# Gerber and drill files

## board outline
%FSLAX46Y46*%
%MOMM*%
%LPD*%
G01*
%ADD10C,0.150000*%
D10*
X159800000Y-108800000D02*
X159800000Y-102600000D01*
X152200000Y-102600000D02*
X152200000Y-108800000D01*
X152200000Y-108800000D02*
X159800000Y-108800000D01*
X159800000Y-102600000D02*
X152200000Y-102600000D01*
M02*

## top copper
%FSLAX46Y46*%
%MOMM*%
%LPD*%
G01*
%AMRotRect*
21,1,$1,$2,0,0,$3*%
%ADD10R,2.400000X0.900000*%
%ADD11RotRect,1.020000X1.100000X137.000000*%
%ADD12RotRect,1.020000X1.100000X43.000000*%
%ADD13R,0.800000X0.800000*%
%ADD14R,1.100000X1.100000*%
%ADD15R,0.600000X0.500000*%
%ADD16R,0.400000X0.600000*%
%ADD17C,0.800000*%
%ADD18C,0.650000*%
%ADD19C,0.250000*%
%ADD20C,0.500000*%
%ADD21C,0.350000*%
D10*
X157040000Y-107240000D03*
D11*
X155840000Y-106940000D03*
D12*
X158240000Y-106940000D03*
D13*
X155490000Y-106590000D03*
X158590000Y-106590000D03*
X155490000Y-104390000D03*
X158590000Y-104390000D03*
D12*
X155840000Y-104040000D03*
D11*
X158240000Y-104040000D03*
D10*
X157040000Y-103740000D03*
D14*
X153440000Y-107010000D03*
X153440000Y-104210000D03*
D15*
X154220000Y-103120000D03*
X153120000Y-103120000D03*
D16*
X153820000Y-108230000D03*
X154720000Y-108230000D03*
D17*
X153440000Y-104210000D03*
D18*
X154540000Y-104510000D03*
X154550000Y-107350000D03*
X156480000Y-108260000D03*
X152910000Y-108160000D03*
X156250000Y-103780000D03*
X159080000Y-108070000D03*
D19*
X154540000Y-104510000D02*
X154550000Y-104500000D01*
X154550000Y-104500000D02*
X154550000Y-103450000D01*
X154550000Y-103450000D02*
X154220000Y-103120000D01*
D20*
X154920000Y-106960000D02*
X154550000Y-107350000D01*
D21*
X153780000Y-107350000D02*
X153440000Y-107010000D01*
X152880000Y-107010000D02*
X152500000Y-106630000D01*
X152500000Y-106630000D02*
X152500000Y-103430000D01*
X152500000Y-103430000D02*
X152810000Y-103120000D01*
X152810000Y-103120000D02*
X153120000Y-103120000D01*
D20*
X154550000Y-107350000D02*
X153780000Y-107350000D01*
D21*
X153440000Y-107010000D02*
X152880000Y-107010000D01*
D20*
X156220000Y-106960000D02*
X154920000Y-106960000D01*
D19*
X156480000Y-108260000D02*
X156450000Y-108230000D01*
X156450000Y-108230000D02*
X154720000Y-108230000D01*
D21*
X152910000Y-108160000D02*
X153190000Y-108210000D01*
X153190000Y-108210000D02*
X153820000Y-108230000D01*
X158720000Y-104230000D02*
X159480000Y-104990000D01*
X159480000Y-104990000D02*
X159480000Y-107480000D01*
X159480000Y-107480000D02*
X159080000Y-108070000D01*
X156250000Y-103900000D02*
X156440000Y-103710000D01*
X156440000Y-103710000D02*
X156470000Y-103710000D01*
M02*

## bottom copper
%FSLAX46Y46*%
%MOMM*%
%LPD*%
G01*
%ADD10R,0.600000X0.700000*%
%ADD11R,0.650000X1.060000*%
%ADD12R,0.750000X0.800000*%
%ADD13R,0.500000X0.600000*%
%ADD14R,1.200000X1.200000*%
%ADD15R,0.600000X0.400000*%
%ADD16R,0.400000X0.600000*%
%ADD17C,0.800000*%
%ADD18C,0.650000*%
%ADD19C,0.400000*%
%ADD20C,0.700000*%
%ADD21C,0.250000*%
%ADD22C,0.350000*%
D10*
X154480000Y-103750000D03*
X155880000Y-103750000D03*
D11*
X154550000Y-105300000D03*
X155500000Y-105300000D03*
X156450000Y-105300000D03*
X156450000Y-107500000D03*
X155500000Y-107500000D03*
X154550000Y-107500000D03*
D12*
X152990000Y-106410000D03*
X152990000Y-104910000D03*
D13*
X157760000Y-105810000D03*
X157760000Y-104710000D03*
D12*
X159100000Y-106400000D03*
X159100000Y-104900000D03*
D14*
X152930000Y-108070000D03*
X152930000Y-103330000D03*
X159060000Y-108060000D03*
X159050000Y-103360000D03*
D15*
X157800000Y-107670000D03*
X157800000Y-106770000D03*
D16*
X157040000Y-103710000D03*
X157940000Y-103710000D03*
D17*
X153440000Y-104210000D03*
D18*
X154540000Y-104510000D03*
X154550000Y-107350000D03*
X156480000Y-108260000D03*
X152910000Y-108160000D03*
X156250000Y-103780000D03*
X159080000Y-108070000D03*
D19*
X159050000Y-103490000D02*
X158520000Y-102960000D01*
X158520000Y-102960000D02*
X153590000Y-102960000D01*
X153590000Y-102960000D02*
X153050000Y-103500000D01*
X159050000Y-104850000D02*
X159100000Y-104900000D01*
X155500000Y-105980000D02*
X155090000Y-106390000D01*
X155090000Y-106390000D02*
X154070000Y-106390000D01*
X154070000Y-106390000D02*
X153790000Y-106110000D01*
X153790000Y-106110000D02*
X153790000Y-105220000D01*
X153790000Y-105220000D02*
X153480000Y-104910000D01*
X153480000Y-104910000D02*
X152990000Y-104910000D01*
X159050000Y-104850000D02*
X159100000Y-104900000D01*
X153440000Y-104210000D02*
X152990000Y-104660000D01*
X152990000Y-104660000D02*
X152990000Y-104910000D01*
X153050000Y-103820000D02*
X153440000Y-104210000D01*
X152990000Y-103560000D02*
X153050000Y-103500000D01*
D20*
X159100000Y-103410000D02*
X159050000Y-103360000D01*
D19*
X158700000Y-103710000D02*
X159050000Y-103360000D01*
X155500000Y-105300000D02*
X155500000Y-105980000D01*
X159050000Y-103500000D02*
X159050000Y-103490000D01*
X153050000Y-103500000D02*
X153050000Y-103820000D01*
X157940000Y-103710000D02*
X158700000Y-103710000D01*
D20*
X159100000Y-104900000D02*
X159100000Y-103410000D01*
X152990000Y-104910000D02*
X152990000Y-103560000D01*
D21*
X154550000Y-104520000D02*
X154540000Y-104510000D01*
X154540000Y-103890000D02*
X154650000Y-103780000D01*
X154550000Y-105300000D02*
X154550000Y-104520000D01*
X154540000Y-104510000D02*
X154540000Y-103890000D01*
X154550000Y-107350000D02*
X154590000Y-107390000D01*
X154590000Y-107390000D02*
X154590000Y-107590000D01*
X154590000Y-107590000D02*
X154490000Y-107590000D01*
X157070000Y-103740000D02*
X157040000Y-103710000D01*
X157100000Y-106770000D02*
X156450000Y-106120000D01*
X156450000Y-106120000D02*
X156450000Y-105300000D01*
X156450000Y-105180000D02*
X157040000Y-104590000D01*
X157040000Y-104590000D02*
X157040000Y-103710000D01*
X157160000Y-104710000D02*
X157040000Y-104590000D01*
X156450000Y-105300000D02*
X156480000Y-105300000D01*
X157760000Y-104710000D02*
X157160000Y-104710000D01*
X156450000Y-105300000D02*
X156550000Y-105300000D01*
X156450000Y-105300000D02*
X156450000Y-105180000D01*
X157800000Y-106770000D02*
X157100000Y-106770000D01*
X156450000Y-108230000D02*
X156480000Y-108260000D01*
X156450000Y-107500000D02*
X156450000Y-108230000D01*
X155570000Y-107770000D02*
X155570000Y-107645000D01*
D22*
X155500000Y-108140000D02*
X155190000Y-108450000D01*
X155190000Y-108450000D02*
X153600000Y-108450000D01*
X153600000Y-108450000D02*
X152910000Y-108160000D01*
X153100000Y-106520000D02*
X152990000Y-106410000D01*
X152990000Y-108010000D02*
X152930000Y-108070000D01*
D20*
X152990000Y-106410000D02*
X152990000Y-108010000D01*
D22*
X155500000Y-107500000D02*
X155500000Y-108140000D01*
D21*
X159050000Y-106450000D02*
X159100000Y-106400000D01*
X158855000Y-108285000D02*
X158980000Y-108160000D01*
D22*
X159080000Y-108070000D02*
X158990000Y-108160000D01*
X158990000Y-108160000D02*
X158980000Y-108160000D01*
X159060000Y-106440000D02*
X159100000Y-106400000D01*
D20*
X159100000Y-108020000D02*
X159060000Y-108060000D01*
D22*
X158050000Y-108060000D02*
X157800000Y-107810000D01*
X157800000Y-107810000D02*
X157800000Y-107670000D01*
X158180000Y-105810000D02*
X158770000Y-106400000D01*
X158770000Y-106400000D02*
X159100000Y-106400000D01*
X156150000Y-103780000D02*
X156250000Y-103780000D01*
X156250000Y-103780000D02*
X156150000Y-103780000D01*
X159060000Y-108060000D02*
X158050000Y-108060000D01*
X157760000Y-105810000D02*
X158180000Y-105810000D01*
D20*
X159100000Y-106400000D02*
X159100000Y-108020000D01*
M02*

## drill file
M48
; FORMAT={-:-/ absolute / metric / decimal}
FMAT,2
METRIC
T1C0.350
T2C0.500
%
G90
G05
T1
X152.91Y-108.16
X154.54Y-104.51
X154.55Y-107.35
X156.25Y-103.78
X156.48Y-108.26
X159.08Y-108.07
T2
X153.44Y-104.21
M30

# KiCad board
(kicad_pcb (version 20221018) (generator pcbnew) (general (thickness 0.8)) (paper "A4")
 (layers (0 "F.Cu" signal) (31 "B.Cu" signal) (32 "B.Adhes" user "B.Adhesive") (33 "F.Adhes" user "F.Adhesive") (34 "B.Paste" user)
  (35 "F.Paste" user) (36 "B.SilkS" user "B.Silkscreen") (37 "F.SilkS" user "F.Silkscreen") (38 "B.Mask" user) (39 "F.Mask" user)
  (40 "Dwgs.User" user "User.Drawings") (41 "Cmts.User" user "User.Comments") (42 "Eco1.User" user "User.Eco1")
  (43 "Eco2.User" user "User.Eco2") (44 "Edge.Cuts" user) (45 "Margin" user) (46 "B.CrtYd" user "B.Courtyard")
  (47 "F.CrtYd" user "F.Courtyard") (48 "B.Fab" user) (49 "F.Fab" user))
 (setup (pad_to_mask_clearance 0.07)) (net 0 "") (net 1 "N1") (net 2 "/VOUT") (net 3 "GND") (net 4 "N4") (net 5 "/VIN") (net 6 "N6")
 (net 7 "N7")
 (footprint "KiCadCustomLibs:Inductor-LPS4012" (layer "F.Cu") (at 157.04 105.49 90)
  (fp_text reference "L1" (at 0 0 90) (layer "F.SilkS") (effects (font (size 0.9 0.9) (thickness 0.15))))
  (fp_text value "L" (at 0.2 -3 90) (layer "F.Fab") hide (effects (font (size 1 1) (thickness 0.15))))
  (pad "1" smd rect (at -1.75 0 90) (size 0.9 2.4) (layers "F.Cu" "F.Paste" "F.Mask") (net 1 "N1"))
  (pad "1" smd rect (at -1.45 -1.2 137) (size 1.02 1.1) (layers "F.Cu" "F.Paste" "F.Mask") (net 1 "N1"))
  (pad "1" smd rect (at -1.45 1.2 43) (size 1.02 1.1) (layers "F.Cu" "F.Paste" "F.Mask") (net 1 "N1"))
  (pad "1" smd rect (at -1.1 -1.55 90) (size 0.8 0.8) (layers "F.Cu" "F.Paste" "F.Mask") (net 1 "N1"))
  (pad "1" smd rect (at -1.1 1.55 90) (size 0.8 0.8) (layers "F.Cu" "F.Paste" "F.Mask") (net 1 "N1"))
  (pad "2" smd rect (at 1.1 -1.55 90) (size 0.8 0.8) (layers "F.Cu" "F.Paste" "F.Mask") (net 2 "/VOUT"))
  (pad "2" smd rect (at 1.1 1.55 90) (size 0.8 0.8) (layers "F.Cu" "F.Paste" "F.Mask") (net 2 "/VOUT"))
  (pad "2" smd rect (at 1.45 -1.2 43) (size 1.02 1.1) (layers "F.Cu" "F.Paste" "F.Mask") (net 2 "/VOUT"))
  (pad "2" smd rect (at 1.45 1.2 137) (size 1.02 1.1) (layers "F.Cu" "F.Paste" "F.Mask") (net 2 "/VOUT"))
  (pad "2" smd rect (at 1.75 0 90) (size 0.9 2.4) (layers "F.Cu" "F.Paste" "F.Mask") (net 2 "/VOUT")))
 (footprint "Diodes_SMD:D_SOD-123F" (layer "F.Cu") (at 153.44 105.61 90)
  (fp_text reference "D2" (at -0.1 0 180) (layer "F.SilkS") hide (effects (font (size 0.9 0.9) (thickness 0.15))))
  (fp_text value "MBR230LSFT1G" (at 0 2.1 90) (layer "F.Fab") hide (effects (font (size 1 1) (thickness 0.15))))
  (pad "1" smd rect (at -1.4 0 90) (size 1.1 1.1) (layers "F.Cu" "F.Paste" "F.Mask") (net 1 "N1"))
  (pad "2" smd rect (at 1.4 0 90) (size 1.1 1.1) (layers "F.Cu" "F.Paste" "F.Mask") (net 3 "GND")))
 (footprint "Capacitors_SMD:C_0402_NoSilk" (layer "F.Cu") (at 153.67 103.12 180)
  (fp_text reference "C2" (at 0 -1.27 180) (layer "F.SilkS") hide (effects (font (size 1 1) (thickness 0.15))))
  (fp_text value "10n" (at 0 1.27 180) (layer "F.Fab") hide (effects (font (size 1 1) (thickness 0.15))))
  (pad "1" smd rect (at -0.55 0 180) (size 0.6 0.5) (layers "F.Cu" "F.Paste" "F.Mask") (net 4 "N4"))
  (pad "2" smd rect (at 0.55 0 180) (size 0.6 0.5) (layers "F.Cu" "F.Paste" "F.Mask") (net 1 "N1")))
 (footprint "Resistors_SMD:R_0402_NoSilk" (layer "F.Cu") (at 154.27 108.23)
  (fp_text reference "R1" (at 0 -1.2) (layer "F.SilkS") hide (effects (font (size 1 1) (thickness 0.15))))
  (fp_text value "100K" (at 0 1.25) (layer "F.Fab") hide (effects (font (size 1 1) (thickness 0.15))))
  (pad "1" smd rect (at -0.45 0) (size 0.4 0.6) (layers "F.Cu" "F.Paste" "F.Mask") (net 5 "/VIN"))
  (pad "2" smd rect (at 0.45 0) (size 0.4 0.6) (layers "F.Cu" "F.Paste" "F.Mask") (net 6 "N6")))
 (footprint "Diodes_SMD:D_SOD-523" (layer "B.Cu") (at 155.18 103.75)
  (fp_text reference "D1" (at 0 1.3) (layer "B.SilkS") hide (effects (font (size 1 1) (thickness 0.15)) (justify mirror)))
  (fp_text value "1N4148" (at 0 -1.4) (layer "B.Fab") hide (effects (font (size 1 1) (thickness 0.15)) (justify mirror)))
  (pad "1" smd rect (at -0.7 0 180) (size 0.6 0.7) (layers "B.Cu" "B.Paste" "B.Mask") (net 4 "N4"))
  (pad "2" smd rect (at 0.7 0 180) (size 0.6 0.7) (layers "B.Cu" "B.Paste" "B.Mask") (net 2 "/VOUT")))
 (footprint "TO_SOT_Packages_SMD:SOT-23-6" (layer "B.Cu") (at 155.5 106.4 -90)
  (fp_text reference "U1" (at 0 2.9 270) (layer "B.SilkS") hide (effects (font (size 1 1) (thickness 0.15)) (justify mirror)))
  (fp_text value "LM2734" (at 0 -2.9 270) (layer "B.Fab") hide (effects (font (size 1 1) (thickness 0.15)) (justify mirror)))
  (pad "1" smd rect (at -1.1 0.95 270) (size 1.06 0.65) (layers "B.Cu" "B.Paste" "B.Mask") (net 4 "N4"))
  (pad "2" smd rect (at -1.1 0 270) (size 1.06 0.65) (layers "B.Cu" "B.Paste" "B.Mask") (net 3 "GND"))
  (pad "3" smd rect (at -1.1 -0.95 270) (size 1.06 0.65) (layers "B.Cu" "B.Paste" "B.Mask") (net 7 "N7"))
  (pad "4" smd rect (at 1.1 -0.95 270) (size 1.06 0.65) (layers "B.Cu" "B.Paste" "B.Mask") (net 6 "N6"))
  (pad "5" smd rect (at 1.1 0 270) (size 1.06 0.65) (layers "B.Cu" "B.Paste" "B.Mask") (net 5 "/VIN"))
  (pad "6" smd rect (at 1.1 0.95 270) (size 1.06 0.65) (layers "B.Cu" "B.Paste" "B.Mask") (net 1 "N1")))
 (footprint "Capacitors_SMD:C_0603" (layer "B.Cu") (at 152.99 105.66 90)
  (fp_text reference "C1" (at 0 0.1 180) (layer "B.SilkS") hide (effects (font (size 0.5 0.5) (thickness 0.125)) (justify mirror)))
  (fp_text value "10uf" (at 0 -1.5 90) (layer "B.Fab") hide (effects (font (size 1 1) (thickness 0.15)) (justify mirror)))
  (pad "1" smd rect (at -0.75 0 90) (size 0.8 0.75) (layers "B.Cu" "B.Paste" "B.Mask") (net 5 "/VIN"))
  (pad "2" smd rect (at 0.75 0 90) (size 0.8 0.75) (layers "B.Cu" "B.Paste" "B.Mask") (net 3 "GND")))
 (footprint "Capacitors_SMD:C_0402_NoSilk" (layer "B.Cu") (at 157.76 105.26 90)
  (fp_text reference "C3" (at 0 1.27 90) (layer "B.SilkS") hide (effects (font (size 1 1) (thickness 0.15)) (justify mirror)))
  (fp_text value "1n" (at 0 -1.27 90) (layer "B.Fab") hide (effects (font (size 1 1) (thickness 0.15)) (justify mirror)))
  (pad "1" smd rect (at -0.55 0 90) (size 0.6 0.5) (layers "B.Cu" "B.Paste" "B.Mask") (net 2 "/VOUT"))
  (pad "2" smd rect (at 0.55 0 90) (size 0.6 0.5) (layers "B.Cu" "B.Paste" "B.Mask") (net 7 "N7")))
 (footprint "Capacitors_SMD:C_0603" (layer "B.Cu") (at 159.1 105.65 90)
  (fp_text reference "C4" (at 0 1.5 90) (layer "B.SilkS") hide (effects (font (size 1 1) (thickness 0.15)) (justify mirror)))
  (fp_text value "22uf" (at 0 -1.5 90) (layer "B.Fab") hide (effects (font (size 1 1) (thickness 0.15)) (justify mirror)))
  (pad "1" smd rect (at -0.75 0 90) (size 0.8 0.75) (layers "B.Cu" "B.Paste" "B.Mask") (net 2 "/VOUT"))
  (pad "2" smd rect (at 0.75 0 90) (size 0.8 0.75) (layers "B.Cu" "B.Paste" "B.Mask") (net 3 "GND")))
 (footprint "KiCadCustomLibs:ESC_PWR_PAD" (layer "B.Cu") (at 152.93 108.07)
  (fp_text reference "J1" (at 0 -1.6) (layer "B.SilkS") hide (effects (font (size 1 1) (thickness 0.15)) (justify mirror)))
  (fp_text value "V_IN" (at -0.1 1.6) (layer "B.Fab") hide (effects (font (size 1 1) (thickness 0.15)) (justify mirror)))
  (pad "1" smd rect (at 0 0) (size 1.2 1.2) (layers "B.Cu" "B.Paste" "B.Mask") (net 5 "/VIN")))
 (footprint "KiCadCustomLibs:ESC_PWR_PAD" (layer "B.Cu") (at 152.93 103.33)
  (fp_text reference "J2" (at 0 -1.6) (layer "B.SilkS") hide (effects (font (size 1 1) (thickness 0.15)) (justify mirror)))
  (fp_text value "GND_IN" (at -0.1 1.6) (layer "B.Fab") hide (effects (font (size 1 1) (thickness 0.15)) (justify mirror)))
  (pad "1" smd rect (at 0 0) (size 1.2 1.2) (layers "B.Cu" "B.Paste" "B.Mask") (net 3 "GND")))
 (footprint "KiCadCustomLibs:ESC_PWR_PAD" (layer "B.Cu") (at 159.06 108.06)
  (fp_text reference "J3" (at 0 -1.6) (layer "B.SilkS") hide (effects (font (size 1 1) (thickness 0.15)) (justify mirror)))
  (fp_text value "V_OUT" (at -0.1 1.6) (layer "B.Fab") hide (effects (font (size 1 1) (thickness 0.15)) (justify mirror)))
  (pad "1" smd rect (at 0 0) (size 1.2 1.2) (layers "B.Cu" "B.Paste" "B.Mask") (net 2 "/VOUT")))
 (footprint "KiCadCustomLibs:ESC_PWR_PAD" (layer "B.Cu") (at 159.05 103.36)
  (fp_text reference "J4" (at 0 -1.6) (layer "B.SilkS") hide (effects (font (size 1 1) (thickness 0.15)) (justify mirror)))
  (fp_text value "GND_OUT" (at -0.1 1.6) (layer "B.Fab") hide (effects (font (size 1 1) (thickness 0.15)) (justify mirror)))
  (pad "1" smd rect (at 0 0) (size 1.2 1.2) (layers "B.Cu" "B.Paste" "B.Mask") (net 3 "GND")))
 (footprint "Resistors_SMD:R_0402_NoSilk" (layer "B.Cu") (at 157.8 107.22 90)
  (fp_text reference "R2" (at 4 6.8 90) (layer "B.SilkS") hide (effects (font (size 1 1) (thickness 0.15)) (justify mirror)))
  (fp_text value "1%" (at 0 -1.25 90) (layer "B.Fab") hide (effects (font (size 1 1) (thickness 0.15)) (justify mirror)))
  (pad "1" smd rect (at -0.45 0 90) (size 0.4 0.6) (layers "B.Cu" "B.Paste" "B.Mask") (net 2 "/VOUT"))
  (pad "2" smd rect (at 0.45 0 90) (size 0.4 0.6) (layers "B.Cu" "B.Paste" "B.Mask") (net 7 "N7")))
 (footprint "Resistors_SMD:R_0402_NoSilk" (layer "B.Cu") (at 157.49 103.71)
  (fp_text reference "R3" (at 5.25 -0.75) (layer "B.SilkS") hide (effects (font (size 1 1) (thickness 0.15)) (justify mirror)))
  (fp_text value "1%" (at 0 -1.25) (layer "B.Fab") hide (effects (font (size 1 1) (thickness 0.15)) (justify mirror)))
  (pad "1" smd rect (at -0.45 0) (size 0.4 0.6) (layers "B.Cu" "B.Paste" "B.Mask") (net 7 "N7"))
  (pad "2" smd rect (at 0.45 0) (size 0.4 0.6) (layers "B.Cu" "B.Paste" "B.Mask") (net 3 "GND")))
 (gr_line (start 159.8 108.8) (end 159.8 102.6) (stroke (width 0.15) (type solid)) (layer "Edge.Cuts"))
 (gr_line (start 152.2 102.6) (end 152.2 108.8) (stroke (width 0.15) (type solid)) (layer "Edge.Cuts"))
 (gr_line (start 152.2 108.8) (end 159.8 108.8) (stroke (width 0.15) (type solid)) (layer "Edge.Cuts"))
 (gr_line (start 159.8 102.6) (end 152.2 102.6) (stroke (width 0.15) (type solid)) (layer "Edge.Cuts"))
 (via (at 153.44 104.21) (size 0.8) (drill 0.5) (layers "F.Cu" "B.Cu") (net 3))
 (segment (start 159.05 103.49) (end 158.52 102.96) (width 0.4) (layer "B.Cu") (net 3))
 (segment (start 158.52 102.96) (end 153.59 102.96) (width 0.4) (layer "B.Cu") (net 3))
 (segment (start 153.59 102.96) (end 153.05 103.5) (width 0.4) (layer "B.Cu") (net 3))
 (segment (start 159.05 104.85) (end 159.1 104.9) (width 0.4) (layer "B.Cu") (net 3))
 (segment (start 155.5 105.98) (end 155.09 106.39) (width 0.4) (layer "B.Cu") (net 3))
 (segment (start 155.09 106.39) (end 154.07 106.39) (width 0.4) (layer "B.Cu") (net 3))
 (segment (start 154.07 106.39) (end 153.79 106.11) (width 0.4) (layer "B.Cu") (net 3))
 (segment (start 153.79 106.11) (end 153.79 105.22) (width 0.4) (layer "B.Cu") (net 3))
 (segment (start 153.79 105.22) (end 153.48 104.91) (width 0.4) (layer "B.Cu") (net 3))
 (segment (start 153.48 104.91) (end 152.99 104.91) (width 0.4) (layer "B.Cu") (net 3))
 (segment (start 159.05 104.85) (end 159.1 104.9) (width 0.4) (layer "B.Cu") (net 3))
 (segment (start 153.44 104.21) (end 152.99 104.66) (width 0.4) (layer "B.Cu") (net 3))
 (segment (start 152.99 104.66) (end 152.99 104.91) (width 0.4) (layer "B.Cu") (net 3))
 (segment (start 153.05 103.82) (end 153.44 104.21) (width 0.4) (layer "B.Cu") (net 3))
 (segment (start 152.99 103.56) (end 153.05 103.5) (width 0.4) (layer "B.Cu") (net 3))
 (segment (start 159.1 103.41) (end 159.05 103.36) (width 0.7) (layer "B.Cu") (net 3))
 (segment (start 158.7 103.71) (end 159.05 103.36) (width 0.4) (layer "B.Cu") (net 3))
 (segment (start 155.5 105.3) (end 155.5 105.98) (width 0.4) (layer "B.Cu") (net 3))
 (segment (start 159.05 103.5) (end 159.05 103.49) (width 0.4) (layer "B.Cu") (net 3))
 (segment (start 153.05 103.5) (end 153.05 103.82) (width 0.4) (layer "B.Cu") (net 3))
 (segment (start 157.94 103.71) (end 158.7 103.71) (width 0.4) (layer "B.Cu") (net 3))
 (segment (start 159.1 104.9) (end 159.1 103.41) (width 0.7) (layer "B.Cu") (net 3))
 (segment (start 152.99 104.91) (end 152.99 103.56) (width 0.7) (layer "B.Cu") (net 3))
 (segment (start 154.54 104.51) (end 154.55 104.5) (width 0.25) (layer "F.Cu") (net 4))
 (segment (start 154.55 104.5) (end 154.55 103.45) (width 0.25) (layer "F.Cu") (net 4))
 (segment (start 154.55 103.45) (end 154.22 103.12) (width 0.25) (layer "F.Cu") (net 4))
 (via (at 154.54 104.51) (size 0.65) (drill 0.35) (layers "F.Cu" "B.Cu") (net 4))
 (segment (start 154.55 104.52) (end 154.54 104.51) (width 0.25) (layer "B.Cu") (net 4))
 (segment (start 154.54 103.89) (end 154.65 103.78) (width 0.25) (layer "B.Cu") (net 4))
 (segment (start 154.55 105.3) (end 154.55 104.52) (width 0.25) (layer "B.Cu") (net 4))
 (segment (start 154.54 104.51) (end 154.54 103.89) (width 0.25) (layer "B.Cu") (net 4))
 (segment (start 154.92 106.96) (end 154.55 107.35) (width 0.5) (layer "F.Cu") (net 1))
 (segment (start 153.78 107.35) (end 153.44 107.01) (width 0.35) (layer "F.Cu") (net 1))
 (segment (start 152.88 107.01) (end 152.5 106.63) (width 0.35) (layer "F.Cu") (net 1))
 (segment (start 152.5 106.63) (end 152.5 103.43) (width 0.35) (layer "F.Cu") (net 1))
 (segment (start 152.5 103.43) (end 152.81 103.12) (width 0.35) (layer "F.Cu") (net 1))
 (segment (start 152.81 103.12) (end 153.12 103.12) (width 0.35) (layer "F.Cu") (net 1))
 (segment (start 154.55 107.35) (end 153.78 107.35) (width 0.5) (layer "F.Cu") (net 1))
 (segment (start 153.44 107.01) (end 152.88 107.01) (width 0.35) (layer "F.Cu") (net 1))
 (segment (start 156.22 106.96) (end 154.92 106.96) (width 0.5) (layer "F.Cu") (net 1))
 (via (at 154.55 107.35) (size 0.65) (drill 0.35) (layers "F.Cu" "B.Cu") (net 1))
 (segment (start 154.55 107.35) (end 154.59 107.39) (width 0.25) (layer "B.Cu") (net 1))
 (segment (start 154.59 107.39) (end 154.59 107.59) (width 0.25) (layer "B.Cu") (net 1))
 (segment (start 154.59 107.59) (end 154.49 107.59) (width 0.25) (layer "B.Cu") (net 1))
 (segment (start 157.07 103.74) (end 157.04 103.71) (width 0.25) (layer "B.Cu") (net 7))
 (segment (start 157.1 106.77) (end 156.45 106.12) (width 0.25) (layer "B.Cu") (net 7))
 (segment (start 156.45 106.12) (end 156.45 105.3) (width 0.25) (layer "B.Cu") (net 7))
 (segment (start 156.45 105.18) (end 157.04 104.59) (width 0.25) (layer "B.Cu") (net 7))
 (segment (start 157.04 104.59) (end 157.04 103.71) (width 0.25) (layer "B.Cu") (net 7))
 (segment (start 157.16 104.71) (end 157.04 104.59) (width 0.25) (layer "B.Cu") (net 7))
 (segment (start 156.45 105.3) (end 156.48 105.3) (width 0.25) (layer "B.Cu") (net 7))
 (segment (start 157.76 104.71) (end 157.16 104.71) (width 0.25) (layer "B.Cu") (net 7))
 (segment (start 156.45 105.3) (end 156.55 105.3) (width 0.25) (layer "B.Cu") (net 7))
 (segment (start 156.45 105.3) (end 156.45 105.18) (width 0.25) (layer "B.Cu") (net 7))
 (segment (start 157.8 106.77) (end 157.1 106.77) (width 0.25) (layer "B.Cu") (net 7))
 (segment (start 156.48 108.26) (end 156.45 108.23) (width 0.25) (layer "F.Cu") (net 6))
 (segment (start 156.45 108.23) (end 154.72 108.23) (width 0.25) (layer "F.Cu") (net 6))
 (via (at 156.48 108.26) (size 0.65) (drill 0.35) (layers "F.Cu" "B.Cu") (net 6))
 (segment (start 156.45 108.23) (end 156.48 108.26) (width 0.25) (layer "B.Cu") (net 6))
 (segment (start 156.45 107.5) (end 156.45 108.23) (width 0.25) (layer "B.Cu") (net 6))
 (segment (start 152.91 108.16) (end 153.19 108.21) (width 0.35) (layer "F.Cu") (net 5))
 (segment (start 153.19 108.21) (end 153.82 108.23) (width 0.35) (layer "F.Cu") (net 5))
 (via (at 152.91 108.16) (size 0.65) (drill 0.35) (layers "F.Cu" "B.Cu") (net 5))
 (segment (start 155.57 107.77) (end 155.57 107.645) (width 0.25) (layer "B.Cu") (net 5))
 (segment (start 155.5 108.14) (end 155.19 108.45) (width 0.35) (layer "B.Cu") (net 5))
 (segment (start 155.19 108.45) (end 153.6 108.45) (width 0.35) (layer "B.Cu") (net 5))
 (segment (start 153.6 108.45) (end 152.91 108.16) (width 0.35) (layer "B.Cu") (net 5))
 (segment (start 153.1 106.52) (end 152.99 106.41) (width 0.35) (layer "B.Cu") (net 5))
 (segment (start 152.99 108.01) (end 152.93 108.07) (width 0.35) (layer "B.Cu") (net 5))
 (segment (start 152.99 106.41) (end 152.99 108.01) (width 0.7) (layer "B.Cu") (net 5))
 (segment (start 155.5 107.5) (end 155.5 108.14) (width 0.35) (layer "B.Cu") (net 5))
 (segment (start 158.72 104.23) (end 159.48 104.99) (width 0.35) (layer "F.Cu") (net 2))
 (segment (start 159.48 104.99) (end 159.48 107.48) (width 0.35) (layer "F.Cu") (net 2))
 (segment (start 159.48 107.48) (end 159.08 108.07) (width 0.35) (layer "F.Cu") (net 2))
 (segment (start 156.25 103.9) (end 156.44 103.71) (width 0.35) (layer "F.Cu") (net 2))
 (segment (start 156.44 103.71) (end 156.47 103.71) (width 0.35) (layer "F.Cu") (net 2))
 (via (at 156.25 103.78) (size 0.65) (drill 0.35) (layers "F.Cu" "B.Cu") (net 2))
 (via (at 159.08 108.07) (size 0.65) (drill 0.35) (layers "F.Cu" "B.Cu") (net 2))
 (segment (start 159.05 106.45) (end 159.1 106.4) (width 0.25) (layer "B.Cu") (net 2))
 (segment (start 158.855 108.285) (end 158.98 108.16) (width 0.25) (layer "B.Cu") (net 2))
 (segment (start 159.08 108.07) (end 158.99 108.16) (width 0.35) (layer "B.Cu") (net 2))
 (segment (start 158.99 108.16) (end 158.98 108.16) (width 0.35) (layer "B.Cu") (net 2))
 (segment (start 159.06 106.44) (end 159.1 106.4) (width 0.35) (layer "B.Cu") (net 2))
 (segment (start 159.1 108.02) (end 159.06 108.06) (width 0.7) (layer "B.Cu") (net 2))
 (segment (start 158.05 108.06) (end 157.8 107.81) (width 0.35) (layer "B.Cu") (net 2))
 (segment (start 157.8 107.81) (end 157.8 107.67) (width 0.35) (layer "B.Cu") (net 2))
 (segment (start 158.18 105.81) (end 158.77 106.4) (width 0.35) (layer "B.Cu") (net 2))
 (segment (start 158.77 106.4) (end 159.1 106.4) (width 0.35) (layer "B.Cu") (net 2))
 (segment (start 156.15 103.78) (end 156.25 103.78) (width 0.35) (layer "B.Cu") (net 2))
 (segment (start 156.25 103.78) (end 156.15 103.78) (width 0.35) (layer "B.Cu") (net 2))
 (segment (start 159.06 108.06) (end 158.05 108.06) (width 0.35) (layer "B.Cu") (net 2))
 (segment (start 157.76 105.81) (end 158.18 105.81) (width 0.35) (layer "B.Cu") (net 2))
 (segment (start 159.1 106.4) (end 159.1 108.02) (width 0.7) (layer "B.Cu") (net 2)))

